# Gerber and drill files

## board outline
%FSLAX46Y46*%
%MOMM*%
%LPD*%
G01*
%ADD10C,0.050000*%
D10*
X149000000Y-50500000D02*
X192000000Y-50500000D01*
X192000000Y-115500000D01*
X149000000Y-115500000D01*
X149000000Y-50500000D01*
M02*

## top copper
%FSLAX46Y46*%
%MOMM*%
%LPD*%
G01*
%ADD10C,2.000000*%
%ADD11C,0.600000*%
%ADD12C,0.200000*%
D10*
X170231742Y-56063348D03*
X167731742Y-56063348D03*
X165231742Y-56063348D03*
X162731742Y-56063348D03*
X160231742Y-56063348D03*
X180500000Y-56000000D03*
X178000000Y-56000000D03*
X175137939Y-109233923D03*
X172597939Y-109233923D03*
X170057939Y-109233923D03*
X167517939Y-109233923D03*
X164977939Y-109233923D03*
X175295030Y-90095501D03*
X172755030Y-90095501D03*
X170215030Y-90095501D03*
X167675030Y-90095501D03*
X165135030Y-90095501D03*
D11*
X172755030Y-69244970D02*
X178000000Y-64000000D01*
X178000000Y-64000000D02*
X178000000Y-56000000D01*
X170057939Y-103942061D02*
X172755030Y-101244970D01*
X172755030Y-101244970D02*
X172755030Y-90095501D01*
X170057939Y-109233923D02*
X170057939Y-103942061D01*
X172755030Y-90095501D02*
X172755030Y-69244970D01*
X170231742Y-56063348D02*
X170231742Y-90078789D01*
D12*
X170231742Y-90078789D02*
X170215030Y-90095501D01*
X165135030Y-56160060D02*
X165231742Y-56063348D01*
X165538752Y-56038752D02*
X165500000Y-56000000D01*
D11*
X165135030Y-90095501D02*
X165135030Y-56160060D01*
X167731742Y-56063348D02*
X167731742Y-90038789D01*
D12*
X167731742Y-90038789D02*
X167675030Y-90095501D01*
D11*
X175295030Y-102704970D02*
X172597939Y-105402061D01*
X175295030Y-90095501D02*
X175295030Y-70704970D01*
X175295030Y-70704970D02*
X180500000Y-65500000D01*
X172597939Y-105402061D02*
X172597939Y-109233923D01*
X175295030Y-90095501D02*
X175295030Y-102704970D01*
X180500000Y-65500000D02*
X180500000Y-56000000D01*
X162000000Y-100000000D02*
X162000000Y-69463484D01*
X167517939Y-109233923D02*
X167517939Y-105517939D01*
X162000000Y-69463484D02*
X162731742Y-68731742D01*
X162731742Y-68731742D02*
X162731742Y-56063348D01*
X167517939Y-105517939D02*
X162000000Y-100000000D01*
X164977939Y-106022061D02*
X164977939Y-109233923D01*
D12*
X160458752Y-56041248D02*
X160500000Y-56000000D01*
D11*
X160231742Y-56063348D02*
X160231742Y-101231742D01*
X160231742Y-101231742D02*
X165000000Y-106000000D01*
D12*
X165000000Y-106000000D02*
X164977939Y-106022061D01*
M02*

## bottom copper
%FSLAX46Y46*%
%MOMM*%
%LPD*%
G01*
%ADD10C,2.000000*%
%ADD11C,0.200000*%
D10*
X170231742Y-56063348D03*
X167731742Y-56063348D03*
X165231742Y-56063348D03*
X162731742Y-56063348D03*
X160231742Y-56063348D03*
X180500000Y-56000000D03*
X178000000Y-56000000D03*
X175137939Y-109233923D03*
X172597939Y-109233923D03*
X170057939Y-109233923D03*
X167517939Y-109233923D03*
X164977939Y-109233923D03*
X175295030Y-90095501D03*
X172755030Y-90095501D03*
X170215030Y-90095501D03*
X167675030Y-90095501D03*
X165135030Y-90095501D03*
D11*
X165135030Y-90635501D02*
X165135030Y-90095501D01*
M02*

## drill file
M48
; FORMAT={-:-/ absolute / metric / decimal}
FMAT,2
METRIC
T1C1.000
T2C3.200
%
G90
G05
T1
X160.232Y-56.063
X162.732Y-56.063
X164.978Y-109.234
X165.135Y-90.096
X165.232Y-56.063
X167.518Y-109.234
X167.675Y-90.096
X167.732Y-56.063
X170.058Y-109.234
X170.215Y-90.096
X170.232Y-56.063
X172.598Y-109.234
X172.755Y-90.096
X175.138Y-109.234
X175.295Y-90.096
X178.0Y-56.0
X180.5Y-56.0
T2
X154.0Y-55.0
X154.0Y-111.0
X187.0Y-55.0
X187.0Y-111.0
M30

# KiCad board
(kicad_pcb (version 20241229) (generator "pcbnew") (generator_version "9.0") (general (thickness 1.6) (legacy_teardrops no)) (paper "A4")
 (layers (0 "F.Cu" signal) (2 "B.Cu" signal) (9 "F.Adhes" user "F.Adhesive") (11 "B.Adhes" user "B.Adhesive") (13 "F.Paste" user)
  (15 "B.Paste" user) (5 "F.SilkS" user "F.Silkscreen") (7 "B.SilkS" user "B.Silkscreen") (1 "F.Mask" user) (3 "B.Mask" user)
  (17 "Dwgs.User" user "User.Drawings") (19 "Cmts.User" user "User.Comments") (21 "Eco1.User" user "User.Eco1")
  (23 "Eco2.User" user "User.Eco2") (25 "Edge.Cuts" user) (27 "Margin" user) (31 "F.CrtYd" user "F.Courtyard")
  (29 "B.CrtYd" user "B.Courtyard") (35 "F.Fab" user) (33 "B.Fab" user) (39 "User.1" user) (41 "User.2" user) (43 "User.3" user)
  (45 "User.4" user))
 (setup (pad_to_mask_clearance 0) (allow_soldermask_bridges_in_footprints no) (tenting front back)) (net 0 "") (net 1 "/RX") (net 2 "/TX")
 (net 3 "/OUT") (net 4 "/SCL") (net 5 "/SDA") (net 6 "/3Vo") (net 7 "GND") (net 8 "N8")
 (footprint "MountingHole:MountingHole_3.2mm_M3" (layer "F.Cu") (at 187 55)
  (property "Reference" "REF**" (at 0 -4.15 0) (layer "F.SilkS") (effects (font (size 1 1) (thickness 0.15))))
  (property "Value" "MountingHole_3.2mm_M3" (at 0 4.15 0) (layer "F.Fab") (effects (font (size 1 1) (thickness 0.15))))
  (pad "" np_thru_hole circle (at 0 0) (size 3.2 3.2) (drill 3.2) (layers "*.Cu" "*.Mask")))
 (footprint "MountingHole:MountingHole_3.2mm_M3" (layer "F.Cu") (at 154 55)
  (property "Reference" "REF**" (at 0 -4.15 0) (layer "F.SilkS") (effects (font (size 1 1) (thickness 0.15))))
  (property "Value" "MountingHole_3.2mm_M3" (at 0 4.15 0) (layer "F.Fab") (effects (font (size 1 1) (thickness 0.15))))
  (pad "" np_thru_hole circle (at 0 0) (size 3.2 3.2) (drill 3.2) (layers "*.Cu" "*.Mask")))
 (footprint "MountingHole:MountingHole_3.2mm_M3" (layer "F.Cu") (at 187 111)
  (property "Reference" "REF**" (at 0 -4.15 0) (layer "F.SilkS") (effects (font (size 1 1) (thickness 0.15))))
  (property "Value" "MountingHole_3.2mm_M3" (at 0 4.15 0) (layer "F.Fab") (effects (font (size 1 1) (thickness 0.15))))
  (pad "" np_thru_hole circle (at 0 0) (size 3.2 3.2) (drill 3.2) (layers "*.Cu" "*.Mask")))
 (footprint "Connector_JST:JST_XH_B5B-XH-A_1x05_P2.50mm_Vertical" (layer "F.Cu") (at 170.231742 56.063348 180)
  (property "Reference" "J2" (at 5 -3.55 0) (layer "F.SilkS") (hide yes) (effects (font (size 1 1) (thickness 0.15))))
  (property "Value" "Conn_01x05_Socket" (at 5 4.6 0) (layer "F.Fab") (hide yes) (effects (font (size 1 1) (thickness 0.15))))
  (pad "1" thru_hole circle (at 0 0 180) (size 2 2) (drill 1) (layers "*.Cu" "*.Mask") (remove_unused_layers no) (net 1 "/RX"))
  (pad "2" thru_hole circle (at 2.5 0 180) (size 2 2) (drill 1) (layers "*.Cu" "*.Mask") (remove_unused_layers no) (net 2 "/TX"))
  (pad "3" thru_hole circle (at 5 0 180) (size 2 2) (drill 1) (layers "*.Cu" "*.Mask") (remove_unused_layers no) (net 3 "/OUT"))
  (pad "4" thru_hole circle (at 7.5 0 180) (size 2 2) (drill 1) (layers "*.Cu" "*.Mask") (remove_unused_layers no) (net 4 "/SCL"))
  (pad "5" thru_hole circle (at 10 0 180) (size 2 2) (drill 1) (layers "*.Cu" "*.Mask") (remove_unused_layers no) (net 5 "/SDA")))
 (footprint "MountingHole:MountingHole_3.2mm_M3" (layer "F.Cu") (at 154 111)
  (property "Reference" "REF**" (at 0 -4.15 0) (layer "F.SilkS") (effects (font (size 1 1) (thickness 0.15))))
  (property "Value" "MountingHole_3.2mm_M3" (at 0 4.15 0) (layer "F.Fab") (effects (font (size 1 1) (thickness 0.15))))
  (pad "" np_thru_hole circle (at 0 0) (size 3.2 3.2) (drill 3.2) (layers "*.Cu" "*.Mask")))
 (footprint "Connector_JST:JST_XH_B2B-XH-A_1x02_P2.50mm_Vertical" (layer "F.Cu") (at 180.5 56 180)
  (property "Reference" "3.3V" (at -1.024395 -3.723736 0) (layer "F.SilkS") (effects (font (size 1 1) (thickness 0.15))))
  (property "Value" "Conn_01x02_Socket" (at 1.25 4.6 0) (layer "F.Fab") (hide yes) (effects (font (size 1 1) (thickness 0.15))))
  (pad "1" thru_hole circle (at 0 0 180) (size 2 2) (drill 1) (layers "*.Cu" "*.Mask") (remove_unused_layers no) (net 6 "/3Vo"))
  (pad "2" thru_hole circle (at 2.5 0 180) (size 2 2) (drill 1) (layers "*.Cu" "*.Mask") (remove_unused_layers no) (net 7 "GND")))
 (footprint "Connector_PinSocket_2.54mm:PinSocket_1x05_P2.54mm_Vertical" (layer "B.Cu") (at 175.137939 109.233923 90)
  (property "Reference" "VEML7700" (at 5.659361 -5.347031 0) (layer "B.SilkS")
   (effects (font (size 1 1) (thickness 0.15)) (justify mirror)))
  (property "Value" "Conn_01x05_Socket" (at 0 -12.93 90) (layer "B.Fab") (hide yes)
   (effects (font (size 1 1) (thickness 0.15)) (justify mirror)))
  (pad "1" thru_hole circle (at 0 0 90) (size 2 2) (drill 1) (layers "*.Cu" "*.Mask") (remove_unused_layers no) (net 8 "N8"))
  (pad "2" thru_hole circle (at 0 -2.54 90) (size 2 2) (drill 1) (layers "*.Cu" "*.Mask") (remove_unused_layers no) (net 6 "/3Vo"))
  (pad "3" thru_hole circle (at 0 -5.08 90) (size 2 2) (drill 1) (layers "*.Cu" "*.Mask") (remove_unused_layers no) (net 7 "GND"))
  (pad "4" thru_hole circle (at 0 -7.62 90) (size 2 2) (drill 1) (layers "*.Cu" "*.Mask") (remove_unused_layers no) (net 4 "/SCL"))
  (pad "5" thru_hole circle (at 0 -10.16 90) (size 2 2) (drill 1) (layers "*.Cu" "*.Mask") (remove_unused_layers no) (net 5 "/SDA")))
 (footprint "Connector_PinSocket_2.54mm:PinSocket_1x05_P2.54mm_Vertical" (layer "B.Cu") (at 175.29503 90.095501 90)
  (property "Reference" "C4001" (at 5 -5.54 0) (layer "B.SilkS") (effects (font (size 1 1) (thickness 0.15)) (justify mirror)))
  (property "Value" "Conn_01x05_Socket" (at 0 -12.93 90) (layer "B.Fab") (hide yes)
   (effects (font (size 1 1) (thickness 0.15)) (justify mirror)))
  (pad "1" thru_hole circle (at 0 0 90) (size 2 2) (drill 1) (layers "*.Cu" "*.Mask") (remove_unused_layers no) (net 6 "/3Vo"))
  (pad "2" thru_hole circle (at 0 -2.54 90) (size 2 2) (drill 1) (layers "*.Cu" "*.Mask") (remove_unused_layers no) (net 7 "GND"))
  (pad "3" thru_hole circle (at 0 -5.08 90) (size 2 2) (drill 1) (layers "*.Cu" "*.Mask") (remove_unused_layers no) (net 1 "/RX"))
  (pad "4" thru_hole circle (at 0 -7.62 90) (size 2 2) (drill 1) (layers "*.Cu" "*.Mask") (remove_unused_layers no) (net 2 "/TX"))
  (pad "5" thru_hole circle (at 0 -10.16 90) (size 2 2) (drill 1) (layers "*.Cu" "*.Mask") (remove_unused_layers no) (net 3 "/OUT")))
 (gr_rect (start 149 50.5) (end 192 115.5) (stroke (width 0.05) (type default)) (fill no) (layer "Edge.Cuts"))
 (segment (start 172.75503 69.24497) (end 178 64) (width 0.6) (layer "F.Cu") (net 7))
 (segment (start 178 64) (end 178 56) (width 0.6) (layer "F.Cu") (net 7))
 (segment (start 170.057939 103.942061) (end 172.75503 101.24497) (width 0.6) (layer "F.Cu") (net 7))
 (segment (start 172.75503 101.24497) (end 172.75503 90.095501) (width 0.6) (layer "F.Cu") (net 7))
 (segment (start 170.057939 109.233923) (end 170.057939 103.942061) (width 0.6) (layer "F.Cu") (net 7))
 (segment (start 172.75503 90.095501) (end 172.75503 69.24497) (width 0.6) (layer "F.Cu") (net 7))
 (segment (start 170.231742 56.063348) (end 170.231742 90.078789) (width 0.6) (layer "F.Cu") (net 1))
 (segment (start 170.231742 90.078789) (end 170.21503 90.095501) (width 0.2) (layer "F.Cu") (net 1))
 (segment (start 165.13503 56.16006) (end 165.231742 56.063348) (width 0.2) (layer "F.Cu") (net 3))
 (segment (start 165.538752 56.038752) (end 165.5 56) (width 0.2) (layer "F.Cu") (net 3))
 (segment (start 165.13503 90.095501) (end 165.13503 56.16006) (width 0.6) (layer "F.Cu") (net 3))
 (segment (start 165.13503 90.635501) (end 165.13503 90.095501) (width 0.2) (layer "B.Cu") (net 3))
 (segment (start 167.731742 56.063348) (end 167.731742 90.038789) (width 0.6) (layer "F.Cu") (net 2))
 (segment (start 167.731742 90.038789) (end 167.67503 90.095501) (width 0.2) (layer "F.Cu") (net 2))
 (segment (start 175.29503 102.70497) (end 172.597939 105.402061) (width 0.6) (layer "F.Cu") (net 6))
 (segment (start 175.29503 90.095501) (end 175.29503 70.70497) (width 0.6) (layer "F.Cu") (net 6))
 (segment (start 175.29503 70.70497) (end 180.5 65.5) (width 0.6) (layer "F.Cu") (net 6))
 (segment (start 172.597939 105.402061) (end 172.597939 109.233923) (width 0.6) (layer "F.Cu") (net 6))
 (segment (start 175.29503 90.095501) (end 175.29503 102.70497) (width 0.6) (layer "F.Cu") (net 6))
 (segment (start 180.5 65.5) (end 180.5 56) (width 0.6) (layer "F.Cu") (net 6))
 (segment (start 162 100) (end 162 69.463484) (width 0.6) (layer "F.Cu") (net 4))
 (segment (start 167.517939 109.233923) (end 167.517939 105.517939) (width 0.6) (layer "F.Cu") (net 4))
 (segment (start 162 69.463484) (end 162.731742 68.731742) (width 0.6) (layer "F.Cu") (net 4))
 (segment (start 162.731742 68.731742) (end 162.731742 56.063348) (width 0.6) (layer "F.Cu") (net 4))
 (segment (start 167.517939 105.517939) (end 162 100) (width 0.6) (layer "F.Cu") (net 4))
 (segment (start 164.977939 106.022061) (end 164.977939 109.233923) (width 0.6) (layer "F.Cu") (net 5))
 (segment (start 160.458752 56.041248) (end 160.5 56) (width 0.2) (layer "F.Cu") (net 5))
 (segment (start 160.231742 56.063348) (end 160.231742 101.231742) (width 0.6) (layer "F.Cu") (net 5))
 (segment (start 160.231742 101.231742) (end 165 106) (width 0.6) (layer "F.Cu") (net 5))
 (segment (start 165 106) (end 164.977939 106.022061) (width 0.2) (layer "F.Cu") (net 5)))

